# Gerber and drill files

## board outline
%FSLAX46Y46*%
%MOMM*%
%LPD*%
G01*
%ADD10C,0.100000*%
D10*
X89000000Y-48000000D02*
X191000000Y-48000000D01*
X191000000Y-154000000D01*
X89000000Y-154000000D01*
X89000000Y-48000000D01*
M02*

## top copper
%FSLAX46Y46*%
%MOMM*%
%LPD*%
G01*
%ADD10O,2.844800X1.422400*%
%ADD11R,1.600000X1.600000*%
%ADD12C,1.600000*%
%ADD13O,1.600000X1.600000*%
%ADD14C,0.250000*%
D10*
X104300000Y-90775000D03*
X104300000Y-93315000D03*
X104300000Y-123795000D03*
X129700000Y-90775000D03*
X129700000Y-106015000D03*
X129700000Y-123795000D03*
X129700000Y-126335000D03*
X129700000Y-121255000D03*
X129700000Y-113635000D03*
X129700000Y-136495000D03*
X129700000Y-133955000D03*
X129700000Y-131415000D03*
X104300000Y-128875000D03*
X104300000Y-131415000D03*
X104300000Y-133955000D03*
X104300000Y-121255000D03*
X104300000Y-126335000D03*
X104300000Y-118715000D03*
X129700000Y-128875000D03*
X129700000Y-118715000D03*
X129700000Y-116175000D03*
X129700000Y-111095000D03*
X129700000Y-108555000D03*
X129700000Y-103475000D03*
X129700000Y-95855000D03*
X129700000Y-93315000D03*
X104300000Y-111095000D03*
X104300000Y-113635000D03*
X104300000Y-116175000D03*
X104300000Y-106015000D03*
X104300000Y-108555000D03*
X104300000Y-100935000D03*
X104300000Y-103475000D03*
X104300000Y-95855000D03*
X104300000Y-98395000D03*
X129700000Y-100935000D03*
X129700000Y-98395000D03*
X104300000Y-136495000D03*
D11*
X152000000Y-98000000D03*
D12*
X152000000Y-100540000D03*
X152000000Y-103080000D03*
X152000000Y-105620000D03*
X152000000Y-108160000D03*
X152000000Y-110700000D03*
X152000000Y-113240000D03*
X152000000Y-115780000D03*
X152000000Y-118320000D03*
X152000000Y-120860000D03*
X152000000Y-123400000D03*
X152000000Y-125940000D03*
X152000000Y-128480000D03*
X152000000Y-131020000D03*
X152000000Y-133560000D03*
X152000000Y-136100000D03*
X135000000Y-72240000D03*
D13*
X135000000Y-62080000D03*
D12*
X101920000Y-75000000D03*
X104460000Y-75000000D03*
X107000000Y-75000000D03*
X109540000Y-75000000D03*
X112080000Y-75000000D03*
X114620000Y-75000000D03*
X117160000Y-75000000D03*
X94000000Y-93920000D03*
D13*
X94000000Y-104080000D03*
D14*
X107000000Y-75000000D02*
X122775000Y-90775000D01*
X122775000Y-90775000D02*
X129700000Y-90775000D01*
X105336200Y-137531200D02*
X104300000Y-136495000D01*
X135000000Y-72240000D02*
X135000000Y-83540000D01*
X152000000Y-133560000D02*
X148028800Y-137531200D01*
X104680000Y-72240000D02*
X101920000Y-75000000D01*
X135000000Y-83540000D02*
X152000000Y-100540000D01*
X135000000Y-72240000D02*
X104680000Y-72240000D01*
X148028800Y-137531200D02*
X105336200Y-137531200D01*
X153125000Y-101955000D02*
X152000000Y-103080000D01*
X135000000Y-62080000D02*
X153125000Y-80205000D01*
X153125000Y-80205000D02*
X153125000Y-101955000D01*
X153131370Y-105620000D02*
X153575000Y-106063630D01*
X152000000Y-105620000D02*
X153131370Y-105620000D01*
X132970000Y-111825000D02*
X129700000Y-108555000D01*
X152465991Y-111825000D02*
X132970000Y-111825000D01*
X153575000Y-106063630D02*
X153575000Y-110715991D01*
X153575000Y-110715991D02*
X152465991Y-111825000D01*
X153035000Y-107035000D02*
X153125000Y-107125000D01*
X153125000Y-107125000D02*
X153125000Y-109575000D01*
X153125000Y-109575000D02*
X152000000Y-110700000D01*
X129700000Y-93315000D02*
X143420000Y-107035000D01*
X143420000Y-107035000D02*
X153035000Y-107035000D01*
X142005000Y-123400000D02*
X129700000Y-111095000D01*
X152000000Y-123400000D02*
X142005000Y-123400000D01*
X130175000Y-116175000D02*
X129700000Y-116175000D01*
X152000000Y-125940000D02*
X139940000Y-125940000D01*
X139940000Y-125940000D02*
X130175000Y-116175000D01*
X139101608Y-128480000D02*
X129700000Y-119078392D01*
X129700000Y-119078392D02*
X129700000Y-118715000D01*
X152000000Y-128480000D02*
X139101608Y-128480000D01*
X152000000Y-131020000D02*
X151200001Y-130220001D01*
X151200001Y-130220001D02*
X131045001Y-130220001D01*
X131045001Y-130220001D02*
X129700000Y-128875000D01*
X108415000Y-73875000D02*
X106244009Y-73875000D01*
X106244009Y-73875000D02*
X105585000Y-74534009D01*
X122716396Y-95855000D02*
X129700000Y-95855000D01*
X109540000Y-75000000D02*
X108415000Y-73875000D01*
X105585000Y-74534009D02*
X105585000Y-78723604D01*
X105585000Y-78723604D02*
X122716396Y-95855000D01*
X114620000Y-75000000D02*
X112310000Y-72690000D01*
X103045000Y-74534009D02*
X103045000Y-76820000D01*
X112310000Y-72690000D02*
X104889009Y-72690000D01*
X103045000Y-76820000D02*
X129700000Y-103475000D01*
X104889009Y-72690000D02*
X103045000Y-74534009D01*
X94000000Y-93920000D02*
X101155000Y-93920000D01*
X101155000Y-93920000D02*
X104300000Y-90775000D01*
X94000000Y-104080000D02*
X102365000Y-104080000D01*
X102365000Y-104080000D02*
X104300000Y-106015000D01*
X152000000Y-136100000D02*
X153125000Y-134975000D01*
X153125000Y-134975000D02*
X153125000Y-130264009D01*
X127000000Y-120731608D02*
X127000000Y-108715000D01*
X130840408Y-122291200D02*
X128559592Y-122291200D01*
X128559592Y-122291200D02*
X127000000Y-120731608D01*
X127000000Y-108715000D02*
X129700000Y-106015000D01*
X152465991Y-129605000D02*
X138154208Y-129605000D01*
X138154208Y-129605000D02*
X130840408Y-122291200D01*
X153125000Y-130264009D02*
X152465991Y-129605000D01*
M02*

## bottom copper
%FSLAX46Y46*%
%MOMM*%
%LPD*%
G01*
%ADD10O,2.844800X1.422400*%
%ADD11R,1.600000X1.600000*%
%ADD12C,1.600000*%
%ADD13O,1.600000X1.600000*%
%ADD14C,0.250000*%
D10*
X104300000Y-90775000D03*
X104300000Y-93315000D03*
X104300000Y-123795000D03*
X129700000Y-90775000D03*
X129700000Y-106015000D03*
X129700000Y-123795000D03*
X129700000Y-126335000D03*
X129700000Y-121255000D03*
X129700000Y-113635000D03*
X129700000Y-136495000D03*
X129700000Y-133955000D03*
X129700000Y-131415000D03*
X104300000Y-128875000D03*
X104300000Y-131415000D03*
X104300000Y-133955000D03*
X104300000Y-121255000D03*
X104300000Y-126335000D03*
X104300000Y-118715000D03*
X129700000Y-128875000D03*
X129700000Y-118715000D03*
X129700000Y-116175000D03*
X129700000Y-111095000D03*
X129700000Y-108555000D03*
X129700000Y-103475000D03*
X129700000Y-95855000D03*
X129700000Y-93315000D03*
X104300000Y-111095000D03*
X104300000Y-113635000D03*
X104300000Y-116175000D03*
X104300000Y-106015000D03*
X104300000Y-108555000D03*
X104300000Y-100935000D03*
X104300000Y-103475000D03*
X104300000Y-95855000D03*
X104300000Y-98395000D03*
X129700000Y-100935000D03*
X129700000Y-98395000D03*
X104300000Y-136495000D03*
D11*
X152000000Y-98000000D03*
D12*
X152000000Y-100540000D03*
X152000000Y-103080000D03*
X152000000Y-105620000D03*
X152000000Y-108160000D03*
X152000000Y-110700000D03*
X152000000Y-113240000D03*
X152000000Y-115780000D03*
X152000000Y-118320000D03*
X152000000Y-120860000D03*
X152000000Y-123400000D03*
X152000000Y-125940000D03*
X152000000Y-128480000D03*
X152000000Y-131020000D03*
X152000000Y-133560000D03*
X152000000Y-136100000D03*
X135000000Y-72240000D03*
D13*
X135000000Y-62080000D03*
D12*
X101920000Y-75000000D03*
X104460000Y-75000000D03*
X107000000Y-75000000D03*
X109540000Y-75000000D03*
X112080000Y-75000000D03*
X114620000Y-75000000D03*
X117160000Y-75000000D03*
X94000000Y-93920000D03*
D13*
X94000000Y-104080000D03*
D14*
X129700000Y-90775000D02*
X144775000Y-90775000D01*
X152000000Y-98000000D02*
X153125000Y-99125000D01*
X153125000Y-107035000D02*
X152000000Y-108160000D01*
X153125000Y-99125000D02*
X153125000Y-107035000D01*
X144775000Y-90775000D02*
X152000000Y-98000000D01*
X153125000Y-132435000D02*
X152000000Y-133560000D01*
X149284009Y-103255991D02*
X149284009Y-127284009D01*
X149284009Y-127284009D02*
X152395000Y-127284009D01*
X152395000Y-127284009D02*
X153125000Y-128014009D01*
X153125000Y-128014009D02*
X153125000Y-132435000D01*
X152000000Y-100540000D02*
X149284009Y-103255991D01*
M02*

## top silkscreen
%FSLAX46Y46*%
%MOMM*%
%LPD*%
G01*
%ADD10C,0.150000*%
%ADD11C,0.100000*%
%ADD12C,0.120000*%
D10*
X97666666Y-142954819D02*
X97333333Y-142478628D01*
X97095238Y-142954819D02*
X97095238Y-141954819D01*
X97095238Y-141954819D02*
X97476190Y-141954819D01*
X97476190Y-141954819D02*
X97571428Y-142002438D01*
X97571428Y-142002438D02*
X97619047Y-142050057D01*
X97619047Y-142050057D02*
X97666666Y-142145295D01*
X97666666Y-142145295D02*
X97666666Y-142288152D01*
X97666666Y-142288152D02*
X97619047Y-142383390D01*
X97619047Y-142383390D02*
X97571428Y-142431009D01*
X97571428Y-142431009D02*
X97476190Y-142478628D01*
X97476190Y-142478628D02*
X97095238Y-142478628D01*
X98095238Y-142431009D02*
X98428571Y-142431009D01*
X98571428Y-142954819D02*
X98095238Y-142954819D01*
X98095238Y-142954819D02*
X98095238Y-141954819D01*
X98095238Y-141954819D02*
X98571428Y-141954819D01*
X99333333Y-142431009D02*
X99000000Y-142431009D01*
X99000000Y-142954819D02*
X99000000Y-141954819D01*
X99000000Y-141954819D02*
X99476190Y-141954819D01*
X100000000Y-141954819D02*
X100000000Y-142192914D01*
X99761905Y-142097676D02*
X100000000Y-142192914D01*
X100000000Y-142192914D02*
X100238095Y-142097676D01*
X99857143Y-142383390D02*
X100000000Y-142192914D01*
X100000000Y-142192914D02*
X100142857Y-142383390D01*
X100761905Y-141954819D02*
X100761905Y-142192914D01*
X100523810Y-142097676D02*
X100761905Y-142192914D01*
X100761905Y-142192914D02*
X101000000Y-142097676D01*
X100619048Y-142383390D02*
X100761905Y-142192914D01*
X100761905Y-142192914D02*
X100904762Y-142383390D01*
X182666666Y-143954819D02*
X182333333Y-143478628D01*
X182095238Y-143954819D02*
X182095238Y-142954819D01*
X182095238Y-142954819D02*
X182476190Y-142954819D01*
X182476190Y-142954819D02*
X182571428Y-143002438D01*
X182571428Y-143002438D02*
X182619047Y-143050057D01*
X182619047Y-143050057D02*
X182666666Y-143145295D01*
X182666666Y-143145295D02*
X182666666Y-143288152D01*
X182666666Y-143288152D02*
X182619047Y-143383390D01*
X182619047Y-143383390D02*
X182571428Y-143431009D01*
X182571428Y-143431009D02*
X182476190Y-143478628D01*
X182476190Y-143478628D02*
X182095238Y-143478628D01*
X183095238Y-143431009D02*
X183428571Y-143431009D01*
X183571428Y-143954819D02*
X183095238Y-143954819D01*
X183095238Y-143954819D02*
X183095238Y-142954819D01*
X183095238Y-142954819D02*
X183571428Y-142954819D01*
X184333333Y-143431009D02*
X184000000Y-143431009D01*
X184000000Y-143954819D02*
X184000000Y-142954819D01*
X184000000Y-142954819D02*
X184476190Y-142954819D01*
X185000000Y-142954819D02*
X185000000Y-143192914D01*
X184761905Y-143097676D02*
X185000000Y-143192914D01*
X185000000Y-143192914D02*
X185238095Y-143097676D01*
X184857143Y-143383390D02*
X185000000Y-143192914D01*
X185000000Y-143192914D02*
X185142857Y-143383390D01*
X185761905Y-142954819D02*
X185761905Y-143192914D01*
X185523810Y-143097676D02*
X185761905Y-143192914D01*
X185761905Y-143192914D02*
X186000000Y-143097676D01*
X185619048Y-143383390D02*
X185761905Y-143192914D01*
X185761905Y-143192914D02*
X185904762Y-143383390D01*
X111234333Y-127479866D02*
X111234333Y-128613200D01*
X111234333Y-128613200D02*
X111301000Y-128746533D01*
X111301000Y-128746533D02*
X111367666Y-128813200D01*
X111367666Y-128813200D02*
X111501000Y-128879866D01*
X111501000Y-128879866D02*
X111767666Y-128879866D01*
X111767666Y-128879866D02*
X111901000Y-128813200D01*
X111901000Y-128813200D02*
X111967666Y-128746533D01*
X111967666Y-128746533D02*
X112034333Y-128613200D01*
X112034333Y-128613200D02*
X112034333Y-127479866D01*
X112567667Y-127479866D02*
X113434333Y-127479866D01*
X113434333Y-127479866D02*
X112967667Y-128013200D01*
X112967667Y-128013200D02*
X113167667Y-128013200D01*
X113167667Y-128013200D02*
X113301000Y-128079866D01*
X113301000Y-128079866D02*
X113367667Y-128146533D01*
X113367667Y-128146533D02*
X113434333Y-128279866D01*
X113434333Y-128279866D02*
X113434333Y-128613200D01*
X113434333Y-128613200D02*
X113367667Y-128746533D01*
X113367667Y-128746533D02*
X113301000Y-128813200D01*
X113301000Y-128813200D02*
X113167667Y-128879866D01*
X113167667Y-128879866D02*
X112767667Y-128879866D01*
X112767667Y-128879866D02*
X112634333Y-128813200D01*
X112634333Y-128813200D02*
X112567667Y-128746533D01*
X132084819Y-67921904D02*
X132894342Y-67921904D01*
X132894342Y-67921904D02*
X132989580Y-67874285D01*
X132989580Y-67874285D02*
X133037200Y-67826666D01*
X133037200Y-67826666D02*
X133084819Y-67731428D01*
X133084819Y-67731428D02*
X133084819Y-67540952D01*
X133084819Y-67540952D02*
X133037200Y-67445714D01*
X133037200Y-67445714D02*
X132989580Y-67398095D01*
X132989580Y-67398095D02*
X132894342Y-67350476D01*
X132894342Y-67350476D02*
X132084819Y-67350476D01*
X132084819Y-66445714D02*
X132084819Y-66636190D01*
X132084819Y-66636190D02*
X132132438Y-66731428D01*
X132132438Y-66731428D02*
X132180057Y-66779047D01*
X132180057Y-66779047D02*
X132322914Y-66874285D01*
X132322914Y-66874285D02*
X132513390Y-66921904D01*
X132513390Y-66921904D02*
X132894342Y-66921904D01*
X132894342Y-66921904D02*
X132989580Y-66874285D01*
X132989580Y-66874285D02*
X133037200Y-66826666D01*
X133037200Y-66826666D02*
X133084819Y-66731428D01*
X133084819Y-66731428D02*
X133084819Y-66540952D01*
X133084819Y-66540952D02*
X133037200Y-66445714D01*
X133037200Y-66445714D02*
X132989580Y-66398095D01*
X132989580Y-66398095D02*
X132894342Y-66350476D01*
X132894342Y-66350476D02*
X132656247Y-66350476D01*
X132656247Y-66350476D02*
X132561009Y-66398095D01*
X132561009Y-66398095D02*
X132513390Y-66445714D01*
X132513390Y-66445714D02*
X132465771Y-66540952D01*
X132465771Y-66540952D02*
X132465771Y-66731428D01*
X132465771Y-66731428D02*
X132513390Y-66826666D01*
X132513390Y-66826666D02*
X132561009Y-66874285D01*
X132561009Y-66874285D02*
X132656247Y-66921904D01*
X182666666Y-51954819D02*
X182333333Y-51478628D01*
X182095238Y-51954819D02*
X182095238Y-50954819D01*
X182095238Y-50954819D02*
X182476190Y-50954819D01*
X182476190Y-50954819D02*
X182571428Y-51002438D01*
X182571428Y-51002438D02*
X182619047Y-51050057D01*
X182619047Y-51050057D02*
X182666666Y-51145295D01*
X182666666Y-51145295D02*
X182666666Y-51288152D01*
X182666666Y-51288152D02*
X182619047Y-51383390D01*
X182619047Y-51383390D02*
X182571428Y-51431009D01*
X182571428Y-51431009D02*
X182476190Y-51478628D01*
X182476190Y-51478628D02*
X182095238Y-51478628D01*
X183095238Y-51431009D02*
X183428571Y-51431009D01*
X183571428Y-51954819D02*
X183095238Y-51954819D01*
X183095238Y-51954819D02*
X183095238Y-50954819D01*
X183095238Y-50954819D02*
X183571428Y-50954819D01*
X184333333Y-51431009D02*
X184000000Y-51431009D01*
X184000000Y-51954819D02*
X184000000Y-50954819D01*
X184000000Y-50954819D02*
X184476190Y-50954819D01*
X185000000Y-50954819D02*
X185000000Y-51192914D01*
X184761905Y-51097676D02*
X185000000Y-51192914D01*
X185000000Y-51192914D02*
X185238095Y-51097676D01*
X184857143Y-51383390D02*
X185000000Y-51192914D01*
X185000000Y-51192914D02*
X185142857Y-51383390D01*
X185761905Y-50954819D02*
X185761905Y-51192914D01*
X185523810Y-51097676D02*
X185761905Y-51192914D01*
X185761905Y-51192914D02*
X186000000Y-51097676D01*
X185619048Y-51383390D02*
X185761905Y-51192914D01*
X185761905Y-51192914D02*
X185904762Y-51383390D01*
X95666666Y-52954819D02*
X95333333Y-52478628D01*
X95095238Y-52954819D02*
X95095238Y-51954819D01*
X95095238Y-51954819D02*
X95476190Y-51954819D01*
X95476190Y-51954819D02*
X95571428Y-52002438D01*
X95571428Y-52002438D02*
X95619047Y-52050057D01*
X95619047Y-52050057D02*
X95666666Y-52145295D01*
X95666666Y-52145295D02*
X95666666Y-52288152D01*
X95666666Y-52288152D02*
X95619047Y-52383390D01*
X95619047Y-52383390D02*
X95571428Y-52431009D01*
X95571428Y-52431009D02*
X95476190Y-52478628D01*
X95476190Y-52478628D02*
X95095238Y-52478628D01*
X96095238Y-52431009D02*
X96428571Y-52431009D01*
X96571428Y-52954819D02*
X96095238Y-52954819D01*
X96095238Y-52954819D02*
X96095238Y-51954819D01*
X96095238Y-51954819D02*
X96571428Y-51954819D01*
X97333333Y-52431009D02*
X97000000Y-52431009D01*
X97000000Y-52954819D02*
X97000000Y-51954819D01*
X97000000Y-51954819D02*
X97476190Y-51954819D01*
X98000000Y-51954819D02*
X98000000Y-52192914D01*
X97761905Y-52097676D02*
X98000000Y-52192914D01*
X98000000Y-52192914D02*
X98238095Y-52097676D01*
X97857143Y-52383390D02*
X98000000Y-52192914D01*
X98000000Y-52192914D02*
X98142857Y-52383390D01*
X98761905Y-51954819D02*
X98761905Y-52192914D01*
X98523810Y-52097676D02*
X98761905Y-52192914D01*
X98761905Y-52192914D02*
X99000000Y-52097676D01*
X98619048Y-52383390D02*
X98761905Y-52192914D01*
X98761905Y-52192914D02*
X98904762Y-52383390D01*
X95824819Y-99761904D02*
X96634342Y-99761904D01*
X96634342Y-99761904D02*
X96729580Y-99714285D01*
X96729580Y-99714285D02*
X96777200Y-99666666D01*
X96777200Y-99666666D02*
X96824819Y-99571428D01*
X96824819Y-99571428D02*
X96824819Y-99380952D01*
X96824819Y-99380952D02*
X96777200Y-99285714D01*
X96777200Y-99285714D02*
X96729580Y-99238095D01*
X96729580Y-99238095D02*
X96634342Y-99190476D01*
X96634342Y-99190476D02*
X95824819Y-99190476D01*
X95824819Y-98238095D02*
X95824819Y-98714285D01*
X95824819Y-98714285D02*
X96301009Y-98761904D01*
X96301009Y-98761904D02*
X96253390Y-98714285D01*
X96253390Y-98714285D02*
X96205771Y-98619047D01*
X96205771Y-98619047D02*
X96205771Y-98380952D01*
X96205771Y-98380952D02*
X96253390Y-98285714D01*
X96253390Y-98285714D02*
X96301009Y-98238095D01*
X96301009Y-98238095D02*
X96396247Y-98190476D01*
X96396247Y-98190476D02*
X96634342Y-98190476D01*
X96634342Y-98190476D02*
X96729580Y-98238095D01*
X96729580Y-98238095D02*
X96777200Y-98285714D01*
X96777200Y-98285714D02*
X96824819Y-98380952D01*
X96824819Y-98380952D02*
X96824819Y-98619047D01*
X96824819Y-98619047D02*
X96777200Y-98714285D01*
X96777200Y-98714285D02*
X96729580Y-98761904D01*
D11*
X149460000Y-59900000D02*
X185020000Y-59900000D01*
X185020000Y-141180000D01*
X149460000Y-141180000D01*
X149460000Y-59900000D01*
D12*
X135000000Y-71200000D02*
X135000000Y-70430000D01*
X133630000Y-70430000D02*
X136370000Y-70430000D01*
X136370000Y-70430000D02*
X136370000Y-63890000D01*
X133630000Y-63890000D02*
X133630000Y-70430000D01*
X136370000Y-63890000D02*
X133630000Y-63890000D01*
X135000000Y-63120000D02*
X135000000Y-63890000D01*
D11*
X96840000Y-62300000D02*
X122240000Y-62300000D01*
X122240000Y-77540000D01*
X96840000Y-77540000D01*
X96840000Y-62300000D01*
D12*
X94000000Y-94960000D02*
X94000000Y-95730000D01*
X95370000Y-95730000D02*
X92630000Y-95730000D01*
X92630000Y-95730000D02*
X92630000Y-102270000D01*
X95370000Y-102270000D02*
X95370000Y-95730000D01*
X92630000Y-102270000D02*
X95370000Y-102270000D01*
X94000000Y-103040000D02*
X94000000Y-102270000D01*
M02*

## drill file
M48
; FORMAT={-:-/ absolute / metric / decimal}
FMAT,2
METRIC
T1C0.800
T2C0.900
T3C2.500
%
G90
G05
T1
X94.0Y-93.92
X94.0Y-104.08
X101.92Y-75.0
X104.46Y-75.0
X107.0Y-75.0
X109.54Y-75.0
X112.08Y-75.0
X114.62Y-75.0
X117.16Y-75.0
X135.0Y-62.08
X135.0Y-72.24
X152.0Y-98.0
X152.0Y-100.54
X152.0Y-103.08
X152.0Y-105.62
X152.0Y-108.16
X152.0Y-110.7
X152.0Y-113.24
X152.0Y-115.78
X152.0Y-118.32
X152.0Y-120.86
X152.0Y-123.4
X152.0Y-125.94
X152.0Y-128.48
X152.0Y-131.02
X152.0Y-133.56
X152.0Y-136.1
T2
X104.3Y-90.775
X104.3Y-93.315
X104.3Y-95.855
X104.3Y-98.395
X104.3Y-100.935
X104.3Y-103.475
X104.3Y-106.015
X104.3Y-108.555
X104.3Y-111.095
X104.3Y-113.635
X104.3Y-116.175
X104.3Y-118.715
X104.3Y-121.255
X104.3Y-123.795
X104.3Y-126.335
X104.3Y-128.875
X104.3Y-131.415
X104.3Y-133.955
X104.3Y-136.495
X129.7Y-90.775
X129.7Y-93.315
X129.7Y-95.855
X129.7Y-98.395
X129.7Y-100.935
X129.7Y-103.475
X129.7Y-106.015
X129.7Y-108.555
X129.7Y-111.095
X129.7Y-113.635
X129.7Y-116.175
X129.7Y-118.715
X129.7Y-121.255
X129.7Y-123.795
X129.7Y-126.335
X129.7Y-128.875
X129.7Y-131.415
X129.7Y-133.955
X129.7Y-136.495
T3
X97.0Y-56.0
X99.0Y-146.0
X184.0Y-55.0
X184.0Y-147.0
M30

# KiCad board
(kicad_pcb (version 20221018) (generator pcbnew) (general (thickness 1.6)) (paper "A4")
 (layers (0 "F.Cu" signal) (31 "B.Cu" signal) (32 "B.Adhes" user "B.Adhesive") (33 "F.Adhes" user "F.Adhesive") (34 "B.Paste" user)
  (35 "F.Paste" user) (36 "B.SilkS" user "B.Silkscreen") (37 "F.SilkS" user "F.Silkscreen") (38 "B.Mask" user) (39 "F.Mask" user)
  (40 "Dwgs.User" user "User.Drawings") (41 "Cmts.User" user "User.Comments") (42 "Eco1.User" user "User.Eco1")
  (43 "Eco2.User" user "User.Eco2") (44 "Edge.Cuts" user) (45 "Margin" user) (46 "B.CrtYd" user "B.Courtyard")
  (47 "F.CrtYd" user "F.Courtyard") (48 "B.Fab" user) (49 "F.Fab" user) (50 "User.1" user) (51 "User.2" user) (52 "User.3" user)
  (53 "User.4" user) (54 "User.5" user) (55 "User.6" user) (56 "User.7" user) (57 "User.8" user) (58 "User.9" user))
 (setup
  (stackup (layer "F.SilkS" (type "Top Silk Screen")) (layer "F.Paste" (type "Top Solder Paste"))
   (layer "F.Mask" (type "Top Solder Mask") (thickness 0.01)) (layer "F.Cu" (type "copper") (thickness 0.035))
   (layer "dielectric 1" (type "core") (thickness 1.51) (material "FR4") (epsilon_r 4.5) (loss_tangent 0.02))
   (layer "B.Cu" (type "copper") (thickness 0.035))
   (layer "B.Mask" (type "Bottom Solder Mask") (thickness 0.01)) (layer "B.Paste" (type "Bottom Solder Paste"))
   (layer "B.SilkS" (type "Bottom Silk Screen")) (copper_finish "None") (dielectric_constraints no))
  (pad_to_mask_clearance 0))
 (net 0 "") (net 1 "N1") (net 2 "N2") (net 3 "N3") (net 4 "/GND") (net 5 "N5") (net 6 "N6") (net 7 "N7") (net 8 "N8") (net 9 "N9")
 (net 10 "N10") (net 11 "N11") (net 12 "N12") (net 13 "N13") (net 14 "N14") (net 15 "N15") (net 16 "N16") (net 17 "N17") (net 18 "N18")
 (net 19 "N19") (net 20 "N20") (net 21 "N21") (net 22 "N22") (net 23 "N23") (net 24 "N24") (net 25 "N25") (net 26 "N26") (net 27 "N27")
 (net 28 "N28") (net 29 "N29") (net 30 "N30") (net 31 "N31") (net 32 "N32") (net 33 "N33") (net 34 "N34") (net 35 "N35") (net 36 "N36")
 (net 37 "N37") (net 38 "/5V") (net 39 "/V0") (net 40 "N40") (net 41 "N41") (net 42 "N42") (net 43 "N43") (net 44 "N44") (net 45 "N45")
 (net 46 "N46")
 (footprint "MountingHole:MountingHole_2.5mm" (layer "F.Cu") (at 99 146)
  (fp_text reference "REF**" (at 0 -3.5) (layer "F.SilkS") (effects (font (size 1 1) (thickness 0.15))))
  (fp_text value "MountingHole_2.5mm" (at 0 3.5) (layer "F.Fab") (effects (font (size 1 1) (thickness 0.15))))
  (pad "" np_thru_hole circle (at 0 0) (size 2.5 2.5) (drill 2.5) (layers "*.Cu" "*.Mask")))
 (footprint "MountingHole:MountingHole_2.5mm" (layer "F.Cu") (at 184 147)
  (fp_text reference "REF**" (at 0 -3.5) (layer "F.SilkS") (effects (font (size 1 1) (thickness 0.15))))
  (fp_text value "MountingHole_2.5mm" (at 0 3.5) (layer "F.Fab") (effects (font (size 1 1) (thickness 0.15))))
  (pad "" np_thru_hole circle (at 0 0) (size 2.5 2.5) (drill 2.5) (layers "*.Cu" "*.Mask")))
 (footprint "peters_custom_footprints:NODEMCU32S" (layer "F.Cu") (at 118.27 112.365)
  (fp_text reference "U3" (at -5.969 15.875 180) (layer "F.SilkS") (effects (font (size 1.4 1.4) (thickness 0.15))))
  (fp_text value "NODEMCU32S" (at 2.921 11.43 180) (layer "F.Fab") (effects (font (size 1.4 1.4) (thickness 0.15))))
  (pad "3V3" thru_hole oval (at -13.97 -21.59) (size 2.8448 1.4224) (drill 0.9) (layers "*.Cu" "*.Mask") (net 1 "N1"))
  (pad "EN" thru_hole oval (at -13.97 -19.05) (size 2.8448 1.4224) (drill 0.9) (layers "*.Cu" "*.Mask") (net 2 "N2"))
  (pad "GND@1" thru_hole oval (at -13.97 11.43) (size 2.8448 1.4224) (drill 0.9) (layers "*.Cu" "*.Mask") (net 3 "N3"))
  (pad "GND@2" thru_hole oval (at 11.43 -21.59) (size 2.8448 1.4224) (drill 0.9) (layers "*.Cu" "*.Mask") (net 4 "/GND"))
  (pad "GND@3" thru_hole oval (at 11.43 -6.35) (size 2.8448 1.4224) (drill 0.9) (layers "*.Cu" "*.Mask") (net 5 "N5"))
  (pad "GPIO0" thru_hole oval (at 11.43 11.43) (size 2.8448 1.4224) (drill 0.9) (layers "*.Cu" "*.Mask") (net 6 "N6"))
  (pad "GPIO2" thru_hole oval (at 11.43 13.97) (size 2.8448 1.4224) (drill 0.9) (layers "*.Cu" "*.Mask") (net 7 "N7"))
  (pad "GPIO4" thru_hole oval (at 11.43 8.89) (size 2.8448 1.4224) (drill 0.9) (layers "*.Cu" "*.Mask") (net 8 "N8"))
  (pad "GPIO5" thru_hole oval (at 11.43 1.27) (size 2.8448 1.4224) (drill 0.9) (layers "*.Cu" "*.Mask") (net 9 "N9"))
  (pad "GPIO6" thru_hole oval (at 11.43 24.13) (size 2.8448 1.4224) (drill 0.9) (layers "*.Cu" "*.Mask") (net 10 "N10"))
  (pad "GPIO7" thru_hole oval (at 11.43 21.59) (size 2.8448 1.4224) (drill 0.9) (layers "*.Cu" "*.Mask") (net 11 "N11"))
  (pad "GPIO8" thru_hole oval (at 11.43 19.05) (size 2.8448 1.4224) (drill 0.9) (layers "*.Cu" "*.Mask") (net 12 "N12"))
  (pad "GPIO9" thru_hole oval (at -13.97 16.51) (size 2.8448 1.4224) (drill 0.9) (layers "*.Cu" "*.Mask") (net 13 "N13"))
  (pad "GPIO10" thru_hole oval (at -13.97 19.05) (size 2.8448 1.4224) (drill 0.9) (layers "*.Cu" "*.Mask") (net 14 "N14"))
  (pad "GPIO11" thru_hole oval (at -13.97 21.59) (size 2.8448 1.4224) (drill 0.9) (layers "*.Cu" "*.Mask") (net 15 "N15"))
  (pad "GPIO12" thru_hole oval (at -13.97 8.89) (size 2.8448 1.4224) (drill 0.9) (layers "*.Cu" "*.Mask") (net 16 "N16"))
  (pad "GPIO13" thru_hole oval (at -13.97 13.97) (size 2.8448 1.4224) (drill 0.9) (layers "*.Cu" "*.Mask") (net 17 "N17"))
  (pad "GPIO14" thru_hole oval (at -13.97 6.35) (size 2.8448 1.4224) (drill 0.9) (layers "*.Cu" "*.Mask") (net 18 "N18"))
  (pad "GPIO15" thru_hole oval (at 11.43 16.51) (size 2.8448 1.4224) (drill 0.9) (layers "*.Cu" "*.Mask") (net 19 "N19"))
  (pad "GPIO16" thru_hole oval (at 11.43 6.35) (size 2.8448 1.4224) (drill 0.9) (layers "*.Cu" "*.Mask") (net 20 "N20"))
  (pad "GPIO17" thru_hole oval (at 11.43 3.81) (size 2.8448 1.4224) (drill 0.9) (layers "*.Cu" "*.Mask") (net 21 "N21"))
  (pad "GPIO18" thru_hole oval (at 11.43 -1.27) (size 2.8448 1.4224) (drill 0.9) (layers "*.Cu" "*.Mask") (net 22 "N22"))
  (pad "GPIO19" thru_hole oval (at 11.43 -3.81) (size 2.8448 1.4224) (drill 0.9) (layers "*.Cu" "*.Mask") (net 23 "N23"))
  (pad "GPIO21" thru_hole oval (at 11.43 -8.89) (size 2.8448 1.4224) (drill 0.9) (layers "*.Cu" "*.Mask") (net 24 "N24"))
  (pad "GPIO22" thru_hole oval (at 11.43 -16.51) (size 2.8448 1.4224) (drill 0.9) (layers "*.Cu" "*.Mask") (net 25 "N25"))
  (pad "GPIO23" thru_hole oval (at 11.43 -19.05) (size 2.8448 1.4224) (drill 0.9) (layers "*.Cu" "*.Mask") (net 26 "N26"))
  (pad "GPIO25" thru_hole oval (at -13.97 -1.27) (size 2.8448 1.4224) (drill 0.9) (layers "*.Cu" "*.Mask") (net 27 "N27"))
  (pad "GPIO26" thru_hole oval (at -13.97 1.27) (size 2.8448 1.4224) (drill 0.9) (layers "*.Cu" "*.Mask") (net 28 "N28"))
  (pad "GPIO27" thru_hole oval (at -13.97 3.81) (size 2.8448 1.4224) (drill 0.9) (layers "*.Cu" "*.Mask") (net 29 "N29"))
  (pad "GPIO32" thru_hole oval (at -13.97 -6.35) (size 2.8448 1.4224) (drill 0.9) (layers "*.Cu" "*.Mask") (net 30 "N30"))
  (pad "GPIO33" thru_hole oval (at -13.97 -3.81) (size 2.8448 1.4224) (drill 0.9) (layers "*.Cu" "*.Mask") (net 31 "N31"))
  (pad "GPIO34" thru_hole oval (at -13.97 -11.43) (size 2.8448 1.4224) (drill 0.9) (layers "*.Cu" "*.Mask") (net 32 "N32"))
  (pad "GPIO35" thru_hole oval (at -13.97 -8.89) (size 2.8448 1.4224) (drill 0.9) (layers "*.Cu" "*.Mask") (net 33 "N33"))
  (pad "GPIO36" thru_hole oval (at -13.97 -16.51) (size 2.8448 1.4224) (drill 0.9) (layers "*.Cu" "*.Mask") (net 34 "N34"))
  (pad "GPIO39" thru_hole oval (at -13.97 -13.97) (size 2.8448 1.4224) (drill 0.9) (layers "*.Cu" "*.Mask") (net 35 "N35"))
  (pad "RX0" thru_hole oval (at 11.43 -11.43) (size 2.8448 1.4224) (drill 0.9) (layers "*.Cu" "*.Mask") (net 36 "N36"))
  (pad "TX0" thru_hole oval (at 11.43 -13.97) (size 2.8448 1.4224) (drill 0.9) (layers "*.Cu" "*.Mask") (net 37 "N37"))
  (pad "VIN" thru_hole oval (at -13.97 24.13) (size 2.8448 1.4224) (drill 0.9) (layers "*.Cu" "*.Mask") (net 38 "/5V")))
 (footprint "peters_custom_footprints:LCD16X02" (layer "F.Cu") (at 98.66 100.54)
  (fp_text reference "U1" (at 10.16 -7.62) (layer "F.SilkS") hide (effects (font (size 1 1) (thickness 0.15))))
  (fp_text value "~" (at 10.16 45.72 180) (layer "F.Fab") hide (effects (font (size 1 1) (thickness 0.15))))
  (fp_rect (start 50.8 -40.64) (end 86.36 40.64) (stroke (width 0.1) (type default)) (fill none) (layer "F.SilkS"))
  (pad "1" thru_hole rect (at 53.34 -2.54 180) (size 1.6 1.6) (drill 0.8) (layers "*.Cu" "*.Mask") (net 4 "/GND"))
  (pad "2" thru_hole circle (at 53.34 0 180) (size 1.6 1.6) (drill 0.8) (layers "*.Cu" "*.Mask") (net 38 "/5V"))
  (pad "3" thru_hole circle (at 53.34 2.54 180) (size 1.6 1.6) (drill 0.8) (layers "*.Cu" "*.Mask") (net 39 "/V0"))
  (pad "4" thru_hole circle (at 53.34 5.08 180) (size 1.6 1.6) (drill 0.8) (layers "*.Cu" "*.Mask") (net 23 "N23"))
  (pad "5" thru_hole circle (at 53.34 7.62 180) (size 1.6 1.6) (drill 0.8) (layers "*.Cu" "*.Mask") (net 4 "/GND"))
  (pad "6" thru_hole circle (at 53.34 10.16 180) (size 1.6 1.6) (drill 0.8) (layers "*.Cu" "*.Mask") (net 26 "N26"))
  (pad "7" thru_hole circle (at 53.34 12.7 180) (size 1.6 1.6) (drill 0.8) (layers "*.Cu" "*.Mask") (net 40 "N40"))
  (pad "8" thru_hole circle (at 53.34 15.24 180) (size 1.6 1.6) (drill 0.8) (layers "*.Cu" "*.Mask") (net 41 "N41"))
  (pad "9" thru_hole circle (at 53.34 17.78 180) (size 1.6 1.6) (drill 0.8) (layers "*.Cu" "*.Mask") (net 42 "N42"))
  (pad "10" thru_hole circle (at 53.34 20.32 180) (size 1.6 1.6) (drill 0.8) (layers "*.Cu" "*.Mask") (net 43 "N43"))
  (pad "11" thru_hole circle (at 53.34 22.86 180) (size 1.6 1.6) (drill 0.8) (layers "*.Cu" "*.Mask") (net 22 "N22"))
  (pad "12" thru_hole circle (at 53.34 25.4 180) (size 1.6 1.6) (drill 0.8) (layers "*.Cu" "*.Mask") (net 21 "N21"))
  (pad "13" thru_hole circle (at 53.34 27.94 180) (size 1.6 1.6) (drill 0.8) (layers "*.Cu" "*.Mask") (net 20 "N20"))
  (pad "14" thru_hole circle (at 53.34 30.48 180) (size 1.6 1.6) (drill 0.8) (layers "*.Cu" "*.Mask") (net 19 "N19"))
  (pad "15" thru_hole circle (at 53.34 33.02 180) (size 1.6 1.6) (drill 0.8) (layers "*.Cu" "*.Mask") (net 38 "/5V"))
  (pad "16" thru_hole circle (at 53.34 35.56 180) (size 1.6 1.6) (drill 0.8) (layers "*.Cu" "*.Mask") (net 5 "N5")))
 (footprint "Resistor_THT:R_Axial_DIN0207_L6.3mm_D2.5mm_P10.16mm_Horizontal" (layer "F.Cu") (at 135 72.24 90)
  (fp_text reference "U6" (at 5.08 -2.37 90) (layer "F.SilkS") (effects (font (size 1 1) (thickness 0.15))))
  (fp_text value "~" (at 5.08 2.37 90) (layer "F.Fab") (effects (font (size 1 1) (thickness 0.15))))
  (fp_line (start 1.04 0) (end 1.81 0) (stroke (width 0.12) (type solid)) (layer "F.SilkS"))
  (fp_line (start 1.81 -1.37) (end 1.81 1.37) (stroke (width 0.12) (type solid)) (layer "F.SilkS"))
  (fp_line (start 1.81 1.37) (end 8.35 1.37) (stroke (width 0.12) (type solid)) (layer "F.SilkS"))
  (fp_line (start 8.35 -1.37) (end 1.81 -1.37) (stroke (width 0.12) (type solid)) (layer "F.SilkS"))
  (fp_line (start 8.35 1.37) (end 8.35 -1.37) (stroke (width 0.12) (type solid)) (layer "F.SilkS"))
  (fp_line (start 9.12 0) (end 8.35 0) (stroke (width 0.12) (type solid)) (layer "F.SilkS"))
  (pad "1" thru_hole circle (at 0 0 90) (size 1.6 1.6) (drill 0.8) (layers "*.Cu" "*.Mask") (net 38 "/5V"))
  (pad "2" thru_hole oval (at 10.16 0 90) (size 1.6 1.6) (drill 0.8) (layers "*.Cu" "*.Mask") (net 39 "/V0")))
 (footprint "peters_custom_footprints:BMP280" (layer "F.Cu") (at 123.41 94.15 -90)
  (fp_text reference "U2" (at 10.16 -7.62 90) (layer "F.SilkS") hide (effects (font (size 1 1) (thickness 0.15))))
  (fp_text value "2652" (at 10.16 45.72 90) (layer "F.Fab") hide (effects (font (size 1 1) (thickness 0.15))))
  (fp_rect (start -16.61 26.57) (end -31.85 1.17) (stroke (width 0.1) (type default)) (fill none) (layer "F.SilkS"))
  (pad "1" thru_hole circle (at -19.15 21.49 270) (size 1.6 1.6) (drill 0.8) (layers "*.Cu" "*.Mask") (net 38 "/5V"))
  (pad "2" thru_hole circle (at -19.15 18.95 270) (size 1.6 1.6) (drill 0.8) (layers "*.Cu" "*.Mask") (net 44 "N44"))
  (pad "3" thru_hole circle (at -19.15 16.41 270) (size 1.6 1.6) (drill 0.8) (layers "*.Cu" "*.Mask") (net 4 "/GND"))
  (pad "4" thru_hole circle (at -19.15 13.87 270) (size 1.6 1.6) (drill 0.8) (layers "*.Cu" "*.Mask") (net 25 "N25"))
  (pad "5" thru_hole circle (at -19.15 11.33 270) (size 1.6 1.6) (drill 0.8) (layers "*.Cu" "*.Mask") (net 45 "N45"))
  (pad "6" thru_hole circle (at -19.15 8.79 270) (size 1.6 1.6) (drill 0.8) (layers "*.Cu" "*.Mask") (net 24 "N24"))
  (pad "7" thru_hole circle (at -19.15 6.25 270) (size 1.6 1.6) (drill 0.8) (layers "*.Cu" "*.Mask") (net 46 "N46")))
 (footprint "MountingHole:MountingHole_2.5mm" (layer "F.Cu") (at 184 55)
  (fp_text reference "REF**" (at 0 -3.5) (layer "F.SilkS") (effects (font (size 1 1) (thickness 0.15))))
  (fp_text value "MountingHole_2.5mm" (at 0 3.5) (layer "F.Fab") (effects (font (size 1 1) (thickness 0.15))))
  (pad "" np_thru_hole circle (at 0 0) (size 2.5 2.5) (drill 2.5) (layers "*.Cu" "*.Mask")))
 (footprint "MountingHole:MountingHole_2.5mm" (layer "F.Cu") (at 97 56)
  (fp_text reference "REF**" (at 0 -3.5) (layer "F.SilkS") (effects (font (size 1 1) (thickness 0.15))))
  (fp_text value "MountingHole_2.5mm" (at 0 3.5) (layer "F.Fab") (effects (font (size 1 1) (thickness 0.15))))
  (pad "" np_thru_hole circle (at 0 0) (size 2.5 2.5) (drill 2.5) (layers "*.Cu" "*.Mask")))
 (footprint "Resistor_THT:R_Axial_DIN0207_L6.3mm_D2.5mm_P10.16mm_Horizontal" (layer "F.Cu") (at 94 93.92 -90)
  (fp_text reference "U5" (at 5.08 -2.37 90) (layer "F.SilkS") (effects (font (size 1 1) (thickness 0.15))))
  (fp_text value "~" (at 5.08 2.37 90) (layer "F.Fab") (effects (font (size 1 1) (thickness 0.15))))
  (fp_line (start 1.04 0) (end 1.81 0) (stroke (width 0.12) (type solid)) (layer "F.SilkS"))
  (fp_line (start 1.81 -1.37) (end 1.81 1.37) (stroke (width 0.12) (type solid)) (layer "F.SilkS"))
  (fp_line (start 1.81 1.37) (end 8.35 1.37) (stroke (width 0.12) (type solid)) (layer "F.SilkS"))
  (fp_line (start 8.35 -1.37) (end 1.81 -1.37) (stroke (width 0.12) (type solid)) (layer "F.SilkS"))
  (fp_line (start 8.35 1.37) (end 8.35 -1.37) (stroke (width 0.12) (type solid)) (layer "F.SilkS"))
  (fp_line (start 9.12 0) (end 8.35 0) (stroke (width 0.12) (type solid)) (layer "F.SilkS"))
  (pad "1" thru_hole circle (at 0 0 270) (size 1.6 1.6) (drill 0.8) (layers "*.Cu" "*.Mask") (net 1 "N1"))
  (pad "2" thru_hole oval (at 10.16 0 270) (size 1.6 1.6) (drill 0.8) (layers "*.Cu" "*.Mask") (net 30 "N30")))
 (gr_rect (start 89 48) (end 191 154) (stroke (width 0.1) (type default)) (fill none) (layer "Edge.Cuts"))
 (segment (start 107 75) (end 122.775 90.775) (width 0.25) (layer "F.Cu") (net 4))
 (segment (start 122.775 90.775) (end 129.7 90.775) (width 0.25) (layer "F.Cu") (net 4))
 (segment (start 129.7 90.775) (end 144.775 90.775) (width 0.25) (layer "B.Cu") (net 4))
 (segment (start 152 98) (end 153.125 99.125) (width 0.25) (layer "B.Cu") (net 4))
 (segment (start 153.125 107.035) (end 152 108.16) (width 0.25) (layer "B.Cu") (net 4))
 (segment (start 153.125 99.125) (end 153.125 107.035) (width 0.25) (layer "B.Cu") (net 4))
 (segment (start 144.775 90.775) (end 152 98) (width 0.25) (layer "B.Cu") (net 4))
 (segment (start 105.3362 137.5312) (end 104.3 136.495) (width 0.25) (layer "F.Cu") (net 38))
 (segment (start 135 72.24) (end 135 83.54) (width 0.25) (layer "F.Cu") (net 38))
 (segment (start 152 133.56) (end 148.0288 137.5312) (width 0.25) (layer "F.Cu") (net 38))
 (segment (start 104.68 72.24) (end 101.92 75) (width 0.25) (layer "F.Cu") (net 38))
 (segment (start 135 83.54) (end 152 100.54) (width 0.25) (layer "F.Cu") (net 38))
 (segment (start 135 72.24) (end 104.68 72.24) (width 0.25) (layer "F.Cu") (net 38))
 (segment (start 148.0288 137.5312) (end 105.3362 137.5312) (width 0.25) (layer "F.Cu") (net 38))
 (segment (start 153.125 132.435) (end 152 133.56) (width 0.25) (layer "B.Cu") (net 38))
 (segment (start 149.284009 103.255991) (end 149.284009 127.284009) (width 0.25) (layer "B.Cu") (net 38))
 (segment (start 149.284009 127.284009) (end 152.395 127.284009) (width 0.25) (layer "B.Cu") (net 38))
 (segment (start 152.395 127.284009) (end 153.125 128.014009) (width 0.25) (layer "B.Cu") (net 38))
 (segment (start 153.125 128.014009) (end 153.125 132.435) (width 0.25) (layer "B.Cu") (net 38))
 (segment (start 152 100.54) (end 149.284009 103.255991) (width 0.25) (layer "B.Cu") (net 38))
 (segment (start 153.125 101.955) (end 152 103.08) (width 0.25) (layer "F.Cu") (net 39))
 (segment (start 135 62.08) (end 153.125 80.205) (width 0.25) (layer "F.Cu") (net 39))
 (segment (start 153.125 80.205) (end 153.125 101.955) (width 0.25) (layer "F.Cu") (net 39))
 (segment (start 153.13137 105.62) (end 153.575 106.06363) (width 0.25) (layer "F.Cu") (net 23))
 (segment (start 152 105.62) (end 153.13137 105.62) (width 0.25) (layer "F.Cu") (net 23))
 (segment (start 132.97 111.825) (end 129.7 108.555) (width 0.25) (layer "F.Cu") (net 23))
 (segment (start 152.465991 111.825) (end 132.97 111.825) (width 0.25) (layer "F.Cu") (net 23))
 (segment (start 153.575 106.06363) (end 153.575 110.715991) (width 0.25) (layer "F.Cu") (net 23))
 (segment (start 153.575 110.715991) (end 152.465991 111.825) (width 0.25) (layer "F.Cu") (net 23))
 (segment (start 153.035 107.035) (end 153.125 107.125) (width 0.25) (layer "F.Cu") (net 26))
 (segment (start 153.125 107.125) (end 153.125 109.575) (width 0.25) (layer "F.Cu") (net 26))
 (segment (start 153.125 109.575) (end 152 110.7) (width 0.25) (layer "F.Cu") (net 26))
 (segment (start 129.7 93.315) (end 143.42 107.035) (width 0.25) (layer "F.Cu") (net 26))
 (segment (start 143.42 107.035) (end 153.035 107.035) (width 0.25) (layer "F.Cu") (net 26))
 (segment (start 142.005 123.4) (end 129.7 111.095) (width 0.25) (layer "F.Cu") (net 22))
 (segment (start 152 123.4) (end 142.005 123.4) (width 0.25) (layer "F.Cu") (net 22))
 (segment (start 130.175 116.175) (end 129.7 116.175) (width 0.25) (layer "F.Cu") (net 21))
 (segment (start 152 125.94) (end 139.94 125.94) (width 0.25) (layer "F.Cu") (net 21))
 (segment (start 139.94 125.94) (end 130.175 116.175) (width 0.25) (layer "F.Cu") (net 21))
 (segment (start 139.101608 128.48) (end 129.7 119.078392) (width 0.25) (layer "F.Cu") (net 20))
 (segment (start 129.7 119.078392) (end 129.7 118.715) (width 0.25) (layer "F.Cu") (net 20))
 (segment (start 152 128.48) (end 139.101608 128.48) (width 0.25) (layer "F.Cu") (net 20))
 (segment (start 152 131.02) (end 151.200001 130.220001) (width 0.25) (layer "F.Cu") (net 19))
 (segment (start 151.200001 130.220001) (end 131.045001 130.220001) (width 0.25) (layer "F.Cu") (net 19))
 (segment (start 131.045001 130.220001) (end 129.7 128.875) (width 0.25) (layer "F.Cu") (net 19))
 (segment (start 108.415 73.875) (end 106.244009 73.875) (width 0.25) (layer "F.Cu") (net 25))
 (segment (start 106.244009 73.875) (end 105.585 74.534009) (width 0.25) (layer "F.Cu") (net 25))
 (segment (start 122.716396 95.855) (end 129.7 95.855) (width 0.25) (layer "F.Cu") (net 25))
 (segment (start 109.54 75) (end 108.415 73.875) (width 0.25) (layer "F.Cu") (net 25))
 (segment (start 105.585 74.534009) (end 105.585 78.723604) (width 0.25) (layer "F.Cu") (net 25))
 (segment (start 105.585 78.723604) (end 122.716396 95.855) (width 0.25) (layer "F.Cu") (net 25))
 (segment (start 114.62 75) (end 112.31 72.69) (width 0.25) (layer "F.Cu") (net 24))
 (segment (start 103.045 74.534009) (end 103.045 76.82) (width 0.25) (layer "F.Cu") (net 24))
 (segment (start 112.31 72.69) (end 104.889009 72.69) (width 0.25) (layer "F.Cu") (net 24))
 (segment (start 103.045 76.82) (end 129.7 103.475) (width 0.25) (layer "F.Cu") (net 24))
 (segment (start 104.889009 72.69) (end 103.045 74.534009) (width 0.25) (layer "F.Cu") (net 24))
 (segment (start 94 93.92) (end 101.155 93.92) (width 0.25) (layer "F.Cu") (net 1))
 (segment (start 101.155 93.92) (end 104.3 90.775) (width 0.25) (layer "F.Cu") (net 1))
 (segment (start 94 104.08) (end 102.365 104.08) (width 0.25) (layer "F.Cu") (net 30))
 (segment (start 102.365 104.08) (end 104.3 106.015) (width 0.25) (layer "F.Cu") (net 30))
 (segment (start 152 136.1) (end 153.125 134.975) (width 0.25) (layer "F.Cu") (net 5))
 (segment (start 153.125 134.975) (end 153.125 130.264009) (width 0.25) (layer "F.Cu") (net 5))
 (segment (start 127 120.731608) (end 127 108.715) (width 0.25) (layer "F.Cu") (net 5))
 (segment (start 130.840408 122.2912) (end 128.559592 122.2912) (width 0.25) (layer "F.Cu") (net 5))
 (segment (start 128.559592 122.2912) (end 127 120.731608) (width 0.25) (layer "F.Cu") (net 5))
 (segment (start 127 108.715) (end 129.7 106.015) (width 0.25) (layer "F.Cu") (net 5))
 (segment (start 152.465991 129.605) (end 138.154208 129.605) (width 0.25) (layer "F.Cu") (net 5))
 (segment (start 138.154208 129.605) (end 130.840408 122.2912) (width 0.25) (layer "F.Cu") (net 5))
 (segment (start 153.125 130.264009) (end 152.465991 129.605) (width 0.25) (layer "F.Cu") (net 5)))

